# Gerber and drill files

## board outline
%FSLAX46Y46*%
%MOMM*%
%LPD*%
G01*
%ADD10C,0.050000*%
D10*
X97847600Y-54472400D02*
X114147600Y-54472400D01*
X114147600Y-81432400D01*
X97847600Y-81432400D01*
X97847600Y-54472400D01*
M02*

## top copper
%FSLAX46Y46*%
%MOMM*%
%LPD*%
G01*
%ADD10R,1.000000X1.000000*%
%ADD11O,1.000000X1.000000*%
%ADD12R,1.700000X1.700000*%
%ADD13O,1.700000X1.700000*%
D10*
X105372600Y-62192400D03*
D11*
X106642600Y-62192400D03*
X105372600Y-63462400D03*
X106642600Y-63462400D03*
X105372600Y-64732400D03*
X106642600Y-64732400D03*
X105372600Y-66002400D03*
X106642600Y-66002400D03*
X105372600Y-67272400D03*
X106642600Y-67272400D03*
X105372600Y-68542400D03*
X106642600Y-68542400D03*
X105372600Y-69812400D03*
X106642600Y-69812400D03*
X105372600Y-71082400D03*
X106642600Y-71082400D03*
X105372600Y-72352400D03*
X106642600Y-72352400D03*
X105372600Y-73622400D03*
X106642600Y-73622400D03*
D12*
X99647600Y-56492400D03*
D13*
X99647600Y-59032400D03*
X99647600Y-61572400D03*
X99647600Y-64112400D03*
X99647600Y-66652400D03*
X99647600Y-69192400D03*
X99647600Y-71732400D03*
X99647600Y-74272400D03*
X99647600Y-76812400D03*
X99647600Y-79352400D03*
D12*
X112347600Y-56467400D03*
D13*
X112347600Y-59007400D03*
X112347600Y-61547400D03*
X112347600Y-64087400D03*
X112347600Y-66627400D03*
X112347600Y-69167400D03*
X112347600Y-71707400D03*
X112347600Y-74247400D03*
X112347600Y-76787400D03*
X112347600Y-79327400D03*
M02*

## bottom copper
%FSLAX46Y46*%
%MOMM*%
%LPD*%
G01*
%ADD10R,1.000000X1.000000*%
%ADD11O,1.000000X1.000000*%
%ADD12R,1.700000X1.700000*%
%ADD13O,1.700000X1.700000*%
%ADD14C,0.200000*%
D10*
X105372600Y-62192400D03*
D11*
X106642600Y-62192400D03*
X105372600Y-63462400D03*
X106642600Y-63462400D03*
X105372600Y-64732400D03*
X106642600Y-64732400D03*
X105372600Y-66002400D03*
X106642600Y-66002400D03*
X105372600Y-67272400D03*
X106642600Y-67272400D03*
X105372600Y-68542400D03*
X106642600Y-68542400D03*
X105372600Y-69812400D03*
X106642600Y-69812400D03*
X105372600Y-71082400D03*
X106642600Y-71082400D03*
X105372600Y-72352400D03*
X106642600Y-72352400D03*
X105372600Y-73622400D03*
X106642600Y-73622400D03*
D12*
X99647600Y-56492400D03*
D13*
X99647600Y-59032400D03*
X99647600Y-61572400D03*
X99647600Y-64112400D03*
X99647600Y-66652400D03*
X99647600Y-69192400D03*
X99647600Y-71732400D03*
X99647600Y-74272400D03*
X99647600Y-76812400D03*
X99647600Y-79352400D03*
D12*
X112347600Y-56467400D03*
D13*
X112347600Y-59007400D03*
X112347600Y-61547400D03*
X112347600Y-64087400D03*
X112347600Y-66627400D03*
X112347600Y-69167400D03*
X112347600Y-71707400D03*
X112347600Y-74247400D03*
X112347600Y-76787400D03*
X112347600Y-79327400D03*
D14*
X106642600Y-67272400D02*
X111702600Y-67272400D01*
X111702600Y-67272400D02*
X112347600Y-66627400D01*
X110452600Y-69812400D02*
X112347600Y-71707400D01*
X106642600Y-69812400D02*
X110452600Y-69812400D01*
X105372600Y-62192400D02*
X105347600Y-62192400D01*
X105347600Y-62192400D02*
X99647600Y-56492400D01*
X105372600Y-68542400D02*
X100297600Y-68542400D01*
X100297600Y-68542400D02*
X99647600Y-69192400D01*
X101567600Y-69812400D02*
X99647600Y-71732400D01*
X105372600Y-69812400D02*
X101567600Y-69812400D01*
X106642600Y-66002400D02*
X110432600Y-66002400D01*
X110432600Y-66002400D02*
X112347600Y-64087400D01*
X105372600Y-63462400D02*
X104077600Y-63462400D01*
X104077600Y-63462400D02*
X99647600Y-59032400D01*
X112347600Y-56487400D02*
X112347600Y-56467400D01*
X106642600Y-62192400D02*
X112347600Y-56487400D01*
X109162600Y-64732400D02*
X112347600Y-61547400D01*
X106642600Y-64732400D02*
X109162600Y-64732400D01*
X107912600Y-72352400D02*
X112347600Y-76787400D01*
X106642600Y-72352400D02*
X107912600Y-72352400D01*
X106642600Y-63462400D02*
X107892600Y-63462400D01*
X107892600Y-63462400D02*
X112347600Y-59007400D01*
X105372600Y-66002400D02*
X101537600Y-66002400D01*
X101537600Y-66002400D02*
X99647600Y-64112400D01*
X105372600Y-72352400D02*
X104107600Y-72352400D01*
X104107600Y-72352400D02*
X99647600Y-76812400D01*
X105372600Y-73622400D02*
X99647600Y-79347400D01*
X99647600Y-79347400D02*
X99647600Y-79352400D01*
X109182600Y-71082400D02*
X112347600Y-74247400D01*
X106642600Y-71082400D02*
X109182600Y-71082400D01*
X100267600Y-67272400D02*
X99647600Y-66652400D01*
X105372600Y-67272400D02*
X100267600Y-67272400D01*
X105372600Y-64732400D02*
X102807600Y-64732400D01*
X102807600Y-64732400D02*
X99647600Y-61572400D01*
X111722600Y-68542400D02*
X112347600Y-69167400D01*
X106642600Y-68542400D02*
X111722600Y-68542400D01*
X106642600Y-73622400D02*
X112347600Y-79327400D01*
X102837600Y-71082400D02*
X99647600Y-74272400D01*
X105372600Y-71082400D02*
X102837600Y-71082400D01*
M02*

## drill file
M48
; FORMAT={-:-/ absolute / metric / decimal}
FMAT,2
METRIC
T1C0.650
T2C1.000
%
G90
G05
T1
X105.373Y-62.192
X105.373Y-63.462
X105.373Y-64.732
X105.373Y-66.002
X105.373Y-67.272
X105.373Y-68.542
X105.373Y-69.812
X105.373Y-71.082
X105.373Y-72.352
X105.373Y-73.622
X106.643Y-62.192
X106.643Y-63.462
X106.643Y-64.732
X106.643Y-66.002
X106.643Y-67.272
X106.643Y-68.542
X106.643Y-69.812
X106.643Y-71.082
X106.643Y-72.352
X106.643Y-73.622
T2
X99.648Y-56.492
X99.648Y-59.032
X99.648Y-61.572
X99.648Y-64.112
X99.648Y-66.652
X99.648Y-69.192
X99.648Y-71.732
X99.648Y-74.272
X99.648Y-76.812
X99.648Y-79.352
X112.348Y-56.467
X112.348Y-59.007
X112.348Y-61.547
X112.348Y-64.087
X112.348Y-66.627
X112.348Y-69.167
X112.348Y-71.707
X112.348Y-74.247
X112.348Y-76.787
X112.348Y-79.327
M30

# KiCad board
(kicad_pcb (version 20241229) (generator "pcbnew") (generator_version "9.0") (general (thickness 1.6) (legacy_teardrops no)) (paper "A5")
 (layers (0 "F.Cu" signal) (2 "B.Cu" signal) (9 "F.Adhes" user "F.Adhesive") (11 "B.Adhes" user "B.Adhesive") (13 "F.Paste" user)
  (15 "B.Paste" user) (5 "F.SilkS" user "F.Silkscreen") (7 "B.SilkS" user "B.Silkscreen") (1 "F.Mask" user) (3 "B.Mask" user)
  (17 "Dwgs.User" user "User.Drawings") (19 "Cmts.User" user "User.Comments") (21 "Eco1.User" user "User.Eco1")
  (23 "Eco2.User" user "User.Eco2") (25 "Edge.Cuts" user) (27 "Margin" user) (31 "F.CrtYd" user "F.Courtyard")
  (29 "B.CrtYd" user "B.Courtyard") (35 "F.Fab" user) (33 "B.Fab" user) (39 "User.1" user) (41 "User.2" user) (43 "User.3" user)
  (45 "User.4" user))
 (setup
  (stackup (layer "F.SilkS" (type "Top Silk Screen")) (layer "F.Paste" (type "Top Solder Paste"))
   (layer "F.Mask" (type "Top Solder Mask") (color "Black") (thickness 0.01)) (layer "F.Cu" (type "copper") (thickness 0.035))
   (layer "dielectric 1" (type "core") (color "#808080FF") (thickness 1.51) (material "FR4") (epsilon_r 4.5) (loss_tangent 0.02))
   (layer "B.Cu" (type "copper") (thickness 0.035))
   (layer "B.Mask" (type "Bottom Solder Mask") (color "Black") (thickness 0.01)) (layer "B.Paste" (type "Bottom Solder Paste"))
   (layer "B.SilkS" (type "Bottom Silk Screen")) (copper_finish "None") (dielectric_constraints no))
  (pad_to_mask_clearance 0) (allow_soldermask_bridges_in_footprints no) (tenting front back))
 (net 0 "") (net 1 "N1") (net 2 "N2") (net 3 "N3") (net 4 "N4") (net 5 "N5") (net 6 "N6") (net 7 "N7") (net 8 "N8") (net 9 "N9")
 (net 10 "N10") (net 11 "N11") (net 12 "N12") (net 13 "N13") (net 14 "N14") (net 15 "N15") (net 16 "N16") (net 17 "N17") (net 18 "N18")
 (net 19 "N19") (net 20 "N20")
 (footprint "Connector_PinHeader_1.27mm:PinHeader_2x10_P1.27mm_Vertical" (layer "F.Cu") (at 105.3726 62.1924)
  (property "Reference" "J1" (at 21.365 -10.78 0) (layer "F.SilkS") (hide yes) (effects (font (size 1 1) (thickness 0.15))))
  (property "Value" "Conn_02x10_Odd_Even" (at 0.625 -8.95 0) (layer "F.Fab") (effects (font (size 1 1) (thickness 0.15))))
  (pad "1" thru_hole rect (at 0 0) (size 1 1) (drill 0.65) (layers "*.Cu" "*.Mask") (remove_unused_layers no) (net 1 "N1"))
  (pad "2" thru_hole oval (at 1.27 0) (size 1 1) (drill 0.65) (layers "*.Cu" "*.Mask") (remove_unused_layers no) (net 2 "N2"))
  (pad "3" thru_hole oval (at 0 1.27) (size 1 1) (drill 0.65) (layers "*.Cu" "*.Mask") (remove_unused_layers no) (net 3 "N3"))
  (pad "4" thru_hole oval (at 1.27 1.27) (size 1 1) (drill 0.65) (layers "*.Cu" "*.Mask") (remove_unused_layers no) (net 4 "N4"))
  (pad "5" thru_hole oval (at 0 2.54) (size 1 1) (drill 0.65) (layers "*.Cu" "*.Mask") (remove_unused_layers no) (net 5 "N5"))
  (pad "6" thru_hole oval (at 1.27 2.54) (size 1 1) (drill 0.65) (layers "*.Cu" "*.Mask") (remove_unused_layers no) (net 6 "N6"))
  (pad "7" thru_hole oval (at 0 3.81) (size 1 1) (drill 0.65) (layers "*.Cu" "*.Mask") (remove_unused_layers no) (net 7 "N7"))
  (pad "8" thru_hole oval (at 1.27 3.81) (size 1 1) (drill 0.65) (layers "*.Cu" "*.Mask") (remove_unused_layers no) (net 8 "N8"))
  (pad "9" thru_hole oval (at 0 5.08) (size 1 1) (drill 0.65) (layers "*.Cu" "*.Mask") (remove_unused_layers no) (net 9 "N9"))
  (pad "10" thru_hole oval (at 1.27 5.08) (size 1 1) (drill 0.65) (layers "*.Cu" "*.Mask") (remove_unused_layers no) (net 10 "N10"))
  (pad "11" thru_hole oval (at 0 6.35) (size 1 1) (drill 0.65) (layers "*.Cu" "*.Mask") (remove_unused_layers no) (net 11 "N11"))
  (pad "12" thru_hole oval (at 1.27 6.35) (size 1 1) (drill 0.65) (layers "*.Cu" "*.Mask") (remove_unused_layers no) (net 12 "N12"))
  (pad "13" thru_hole oval (at 0 7.62) (size 1 1) (drill 0.65) (layers "*.Cu" "*.Mask") (remove_unused_layers no) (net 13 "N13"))
  (pad "14" thru_hole oval (at 1.27 7.62) (size 1 1) (drill 0.65) (layers "*.Cu" "*.Mask") (remove_unused_layers no) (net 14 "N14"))
  (pad "15" thru_hole oval (at 0 8.89) (size 1 1) (drill 0.65) (layers "*.Cu" "*.Mask") (remove_unused_layers no) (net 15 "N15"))
  (pad "16" thru_hole oval (at 1.27 8.89) (size 1 1) (drill 0.65) (layers "*.Cu" "*.Mask") (remove_unused_layers no) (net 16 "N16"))
  (pad "17" thru_hole oval (at 0 10.16) (size 1 1) (drill 0.65) (layers "*.Cu" "*.Mask") (remove_unused_layers no) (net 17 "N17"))
  (pad "18" thru_hole oval (at 1.27 10.16) (size 1 1) (drill 0.65) (layers "*.Cu" "*.Mask") (remove_unused_layers no) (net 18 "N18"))
  (pad "19" thru_hole oval (at 0 11.43) (size 1 1) (drill 0.65) (layers "*.Cu" "*.Mask") (remove_unused_layers no) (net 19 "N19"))
  (pad "20" thru_hole oval (at 1.27 11.43) (size 1 1) (drill 0.65) (layers "*.Cu" "*.Mask") (remove_unused_layers no) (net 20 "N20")))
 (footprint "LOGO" (layer "F.Cu") (at 106.0704 77.978 90)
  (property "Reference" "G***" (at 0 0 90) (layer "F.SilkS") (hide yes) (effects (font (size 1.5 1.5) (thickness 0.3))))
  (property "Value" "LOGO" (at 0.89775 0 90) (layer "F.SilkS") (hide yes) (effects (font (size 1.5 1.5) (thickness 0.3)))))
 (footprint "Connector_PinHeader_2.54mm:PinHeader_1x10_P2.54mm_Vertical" (layer "B.Cu") (at 99.6476 56.4924 180)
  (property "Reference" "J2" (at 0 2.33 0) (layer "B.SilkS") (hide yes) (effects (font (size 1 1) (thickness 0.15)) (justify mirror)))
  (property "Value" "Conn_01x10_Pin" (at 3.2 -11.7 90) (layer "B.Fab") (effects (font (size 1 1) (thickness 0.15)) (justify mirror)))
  (pad "1" thru_hole rect (at 0 0 180) (size 1.7 1.7) (drill 1) (layers "*.Cu" "*.Mask") (remove_unused_layers no) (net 1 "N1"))
  (pad "2" thru_hole oval (at 0 -2.54 180) (size 1.7 1.7) (drill 1) (layers "*.Cu" "*.Mask") (remove_unused_layers no) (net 3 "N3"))
  (pad "3" thru_hole oval (at 0 -5.08 180) (size 1.7 1.7) (drill 1) (layers "*.Cu" "*.Mask") (remove_unused_layers no) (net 5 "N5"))
  (pad "4" thru_hole oval (at 0 -7.62 180) (size 1.7 1.7) (drill 1) (layers "*.Cu" "*.Mask") (remove_unused_layers no) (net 7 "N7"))
  (pad "5" thru_hole oval (at 0 -10.16 180) (size 1.7 1.7) (drill 1) (layers "*.Cu" "*.Mask") (remove_unused_layers no) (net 9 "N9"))
  (pad "6" thru_hole oval (at 0 -12.7 180) (size 1.7 1.7) (drill 1) (layers "*.Cu" "*.Mask") (remove_unused_layers no) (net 11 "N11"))
  (pad "7" thru_hole oval (at 0 -15.24 180) (size 1.7 1.7) (drill 1) (layers "*.Cu" "*.Mask") (remove_unused_layers no) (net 13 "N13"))
  (pad "8" thru_hole oval (at 0 -17.78 180) (size 1.7 1.7) (drill 1) (layers "*.Cu" "*.Mask") (remove_unused_layers no) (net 15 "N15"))
  (pad "9" thru_hole oval (at 0 -20.32 180) (size 1.7 1.7) (drill 1) (layers "*.Cu" "*.Mask") (remove_unused_layers no) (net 17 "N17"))
  (pad "10" thru_hole oval (at 0 -22.86 180) (size 1.7 1.7) (drill 1) (layers "*.Cu" "*.Mask") (remove_unused_layers no) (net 19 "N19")))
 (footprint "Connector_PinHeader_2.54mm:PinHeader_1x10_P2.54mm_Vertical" (layer "B.Cu") (at 112.3476 56.4674 180)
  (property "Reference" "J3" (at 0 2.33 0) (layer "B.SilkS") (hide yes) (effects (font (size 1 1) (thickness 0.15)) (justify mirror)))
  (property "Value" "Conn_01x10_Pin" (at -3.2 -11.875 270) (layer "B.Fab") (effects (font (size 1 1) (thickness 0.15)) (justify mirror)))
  (pad "1" thru_hole rect (at 0 0 180) (size 1.7 1.7) (drill 1) (layers "*.Cu" "*.Mask") (remove_unused_layers no) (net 2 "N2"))
  (pad "2" thru_hole oval (at 0 -2.54 180) (size 1.7 1.7) (drill 1) (layers "*.Cu" "*.Mask") (remove_unused_layers no) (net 4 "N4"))
  (pad "3" thru_hole oval (at 0 -5.08 180) (size 1.7 1.7) (drill 1) (layers "*.Cu" "*.Mask") (remove_unused_layers no) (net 6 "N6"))
  (pad "4" thru_hole oval (at 0 -7.62 180) (size 1.7 1.7) (drill 1) (layers "*.Cu" "*.Mask") (remove_unused_layers no) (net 8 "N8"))
  (pad "5" thru_hole oval (at 0 -10.16 180) (size 1.7 1.7) (drill 1) (layers "*.Cu" "*.Mask") (remove_unused_layers no) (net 10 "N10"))
  (pad "6" thru_hole oval (at 0 -12.7 180) (size 1.7 1.7) (drill 1) (layers "*.Cu" "*.Mask") (remove_unused_layers no) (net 12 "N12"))
  (pad "7" thru_hole oval (at 0 -15.24 180) (size 1.7 1.7) (drill 1) (layers "*.Cu" "*.Mask") (remove_unused_layers no) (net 14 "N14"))
  (pad "8" thru_hole oval (at 0 -17.78 180) (size 1.7 1.7) (drill 1) (layers "*.Cu" "*.Mask") (remove_unused_layers no) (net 16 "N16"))
  (pad "9" thru_hole oval (at 0 -20.32 180) (size 1.7 1.7) (drill 1) (layers "*.Cu" "*.Mask") (remove_unused_layers no) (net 18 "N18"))
  (pad "10" thru_hole oval (at 0 -22.86 180) (size 1.7 1.7) (drill 1) (layers "*.Cu" "*.Mask") (remove_unused_layers no) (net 20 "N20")))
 (gr_rect (start 97.8476 54.4724) (end 114.1476 81.4324) (stroke (width 0.05) (type default)) (fill no) (layer "Edge.Cuts"))
 (segment (start 106.6426 67.2724) (end 111.7026 67.2724) (width 0.2) (layer "B.Cu") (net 10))
 (segment (start 111.7026 67.2724) (end 112.3476 66.6274) (width 0.2) (layer "B.Cu") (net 10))
 (segment (start 110.4526 69.8124) (end 112.3476 71.7074) (width 0.2) (layer "B.Cu") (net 14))
 (segment (start 106.6426 69.8124) (end 110.4526 69.8124) (width 0.2) (layer "B.Cu") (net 14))
 (segment (start 105.3726 62.1924) (end 105.3476 62.1924) (width 0.2) (layer "B.Cu") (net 1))
 (segment (start 105.3476 62.1924) (end 99.6476 56.4924) (width 0.2) (layer "B.Cu") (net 1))
 (segment (start 105.3726 68.5424) (end 100.2976 68.5424) (width 0.2) (layer "B.Cu") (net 11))
 (segment (start 100.2976 68.5424) (end 99.6476 69.1924) (width 0.2) (layer "B.Cu") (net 11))
 (segment (start 101.5676 69.8124) (end 99.6476 71.7324) (width 0.2) (layer "B.Cu") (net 13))
 (segment (start 105.3726 69.8124) (end 101.5676 69.8124) (width 0.2) (layer "B.Cu") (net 13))
 (segment (start 106.6426 66.0024) (end 110.4326 66.0024) (width 0.2) (layer "B.Cu") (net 8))
 (segment (start 110.4326 66.0024) (end 112.3476 64.0874) (width 0.2) (layer "B.Cu") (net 8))
 (segment (start 105.3726 63.4624) (end 104.0776 63.4624) (width 0.2) (layer "B.Cu") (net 3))
 (segment (start 104.0776 63.4624) (end 99.6476 59.0324) (width 0.2) (layer "B.Cu") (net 3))
 (segment (start 112.3476 56.4874) (end 112.3476 56.4674) (width 0.2) (layer "B.Cu") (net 2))
 (segment (start 106.6426 62.1924) (end 112.3476 56.4874) (width 0.2) (layer "B.Cu") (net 2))
 (segment (start 109.1626 64.7324) (end 112.3476 61.5474) (width 0.2) (layer "B.Cu") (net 6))
 (segment (start 106.6426 64.7324) (end 109.1626 64.7324) (width 0.2) (layer "B.Cu") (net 6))
 (segment (start 107.9126 72.3524) (end 112.3476 76.7874) (width 0.2) (layer "B.Cu") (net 18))
 (segment (start 106.6426 72.3524) (end 107.9126 72.3524) (width 0.2) (layer "B.Cu") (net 18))
 (segment (start 106.6426 63.4624) (end 107.8926 63.4624) (width 0.2) (layer "B.Cu") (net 4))
 (segment (start 107.8926 63.4624) (end 112.3476 59.0074) (width 0.2) (layer "B.Cu") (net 4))
 (segment (start 105.3726 66.0024) (end 101.5376 66.0024) (width 0.2) (layer "B.Cu") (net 7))
 (segment (start 101.5376 66.0024) (end 99.6476 64.1124) (width 0.2) (layer "B.Cu") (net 7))
 (segment (start 105.3726 72.3524) (end 104.1076 72.3524) (width 0.2) (layer "B.Cu") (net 17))
 (segment (start 104.1076 72.3524) (end 99.6476 76.8124) (width 0.2) (layer "B.Cu") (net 17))
 (segment (start 105.3726 73.6224) (end 99.6476 79.3474) (width 0.2) (layer "B.Cu") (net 19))
 (segment (start 99.6476 79.3474) (end 99.6476 79.3524) (width 0.2) (layer "B.Cu") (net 19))
 (segment (start 109.1826 71.0824) (end 112.3476 74.2474) (width 0.2) (layer "B.Cu") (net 16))
 (segment (start 106.6426 71.0824) (end 109.1826 71.0824) (width 0.2) (layer "B.Cu") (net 16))
 (segment (start 100.2676 67.2724) (end 99.6476 66.6524) (width 0.2) (layer "B.Cu") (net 9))
 (segment (start 105.3726 67.2724) (end 100.2676 67.2724) (width 0.2) (layer "B.Cu") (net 9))
 (segment (start 105.3726 64.7324) (end 102.8076 64.7324) (width 0.2) (layer "B.Cu") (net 5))
 (segment (start 102.8076 64.7324) (end 99.6476 61.5724) (width 0.2) (layer "B.Cu") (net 5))
 (segment (start 111.7226 68.5424) (end 112.3476 69.1674) (width 0.2) (layer "B.Cu") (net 12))
 (segment (start 106.6426 68.5424) (end 111.7226 68.5424) (width 0.2) (layer "B.Cu") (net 12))
 (segment (start 106.6426 73.6224) (end 112.3476 79.3274) (width 0.2) (layer "B.Cu") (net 20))
 (segment (start 102.8376 71.0824) (end 99.6476 74.2724) (width 0.2) (layer "B.Cu") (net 15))
 (segment (start 105.3726 71.0824) (end 102.8376 71.0824) (width 0.2) (layer "B.Cu") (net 15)))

